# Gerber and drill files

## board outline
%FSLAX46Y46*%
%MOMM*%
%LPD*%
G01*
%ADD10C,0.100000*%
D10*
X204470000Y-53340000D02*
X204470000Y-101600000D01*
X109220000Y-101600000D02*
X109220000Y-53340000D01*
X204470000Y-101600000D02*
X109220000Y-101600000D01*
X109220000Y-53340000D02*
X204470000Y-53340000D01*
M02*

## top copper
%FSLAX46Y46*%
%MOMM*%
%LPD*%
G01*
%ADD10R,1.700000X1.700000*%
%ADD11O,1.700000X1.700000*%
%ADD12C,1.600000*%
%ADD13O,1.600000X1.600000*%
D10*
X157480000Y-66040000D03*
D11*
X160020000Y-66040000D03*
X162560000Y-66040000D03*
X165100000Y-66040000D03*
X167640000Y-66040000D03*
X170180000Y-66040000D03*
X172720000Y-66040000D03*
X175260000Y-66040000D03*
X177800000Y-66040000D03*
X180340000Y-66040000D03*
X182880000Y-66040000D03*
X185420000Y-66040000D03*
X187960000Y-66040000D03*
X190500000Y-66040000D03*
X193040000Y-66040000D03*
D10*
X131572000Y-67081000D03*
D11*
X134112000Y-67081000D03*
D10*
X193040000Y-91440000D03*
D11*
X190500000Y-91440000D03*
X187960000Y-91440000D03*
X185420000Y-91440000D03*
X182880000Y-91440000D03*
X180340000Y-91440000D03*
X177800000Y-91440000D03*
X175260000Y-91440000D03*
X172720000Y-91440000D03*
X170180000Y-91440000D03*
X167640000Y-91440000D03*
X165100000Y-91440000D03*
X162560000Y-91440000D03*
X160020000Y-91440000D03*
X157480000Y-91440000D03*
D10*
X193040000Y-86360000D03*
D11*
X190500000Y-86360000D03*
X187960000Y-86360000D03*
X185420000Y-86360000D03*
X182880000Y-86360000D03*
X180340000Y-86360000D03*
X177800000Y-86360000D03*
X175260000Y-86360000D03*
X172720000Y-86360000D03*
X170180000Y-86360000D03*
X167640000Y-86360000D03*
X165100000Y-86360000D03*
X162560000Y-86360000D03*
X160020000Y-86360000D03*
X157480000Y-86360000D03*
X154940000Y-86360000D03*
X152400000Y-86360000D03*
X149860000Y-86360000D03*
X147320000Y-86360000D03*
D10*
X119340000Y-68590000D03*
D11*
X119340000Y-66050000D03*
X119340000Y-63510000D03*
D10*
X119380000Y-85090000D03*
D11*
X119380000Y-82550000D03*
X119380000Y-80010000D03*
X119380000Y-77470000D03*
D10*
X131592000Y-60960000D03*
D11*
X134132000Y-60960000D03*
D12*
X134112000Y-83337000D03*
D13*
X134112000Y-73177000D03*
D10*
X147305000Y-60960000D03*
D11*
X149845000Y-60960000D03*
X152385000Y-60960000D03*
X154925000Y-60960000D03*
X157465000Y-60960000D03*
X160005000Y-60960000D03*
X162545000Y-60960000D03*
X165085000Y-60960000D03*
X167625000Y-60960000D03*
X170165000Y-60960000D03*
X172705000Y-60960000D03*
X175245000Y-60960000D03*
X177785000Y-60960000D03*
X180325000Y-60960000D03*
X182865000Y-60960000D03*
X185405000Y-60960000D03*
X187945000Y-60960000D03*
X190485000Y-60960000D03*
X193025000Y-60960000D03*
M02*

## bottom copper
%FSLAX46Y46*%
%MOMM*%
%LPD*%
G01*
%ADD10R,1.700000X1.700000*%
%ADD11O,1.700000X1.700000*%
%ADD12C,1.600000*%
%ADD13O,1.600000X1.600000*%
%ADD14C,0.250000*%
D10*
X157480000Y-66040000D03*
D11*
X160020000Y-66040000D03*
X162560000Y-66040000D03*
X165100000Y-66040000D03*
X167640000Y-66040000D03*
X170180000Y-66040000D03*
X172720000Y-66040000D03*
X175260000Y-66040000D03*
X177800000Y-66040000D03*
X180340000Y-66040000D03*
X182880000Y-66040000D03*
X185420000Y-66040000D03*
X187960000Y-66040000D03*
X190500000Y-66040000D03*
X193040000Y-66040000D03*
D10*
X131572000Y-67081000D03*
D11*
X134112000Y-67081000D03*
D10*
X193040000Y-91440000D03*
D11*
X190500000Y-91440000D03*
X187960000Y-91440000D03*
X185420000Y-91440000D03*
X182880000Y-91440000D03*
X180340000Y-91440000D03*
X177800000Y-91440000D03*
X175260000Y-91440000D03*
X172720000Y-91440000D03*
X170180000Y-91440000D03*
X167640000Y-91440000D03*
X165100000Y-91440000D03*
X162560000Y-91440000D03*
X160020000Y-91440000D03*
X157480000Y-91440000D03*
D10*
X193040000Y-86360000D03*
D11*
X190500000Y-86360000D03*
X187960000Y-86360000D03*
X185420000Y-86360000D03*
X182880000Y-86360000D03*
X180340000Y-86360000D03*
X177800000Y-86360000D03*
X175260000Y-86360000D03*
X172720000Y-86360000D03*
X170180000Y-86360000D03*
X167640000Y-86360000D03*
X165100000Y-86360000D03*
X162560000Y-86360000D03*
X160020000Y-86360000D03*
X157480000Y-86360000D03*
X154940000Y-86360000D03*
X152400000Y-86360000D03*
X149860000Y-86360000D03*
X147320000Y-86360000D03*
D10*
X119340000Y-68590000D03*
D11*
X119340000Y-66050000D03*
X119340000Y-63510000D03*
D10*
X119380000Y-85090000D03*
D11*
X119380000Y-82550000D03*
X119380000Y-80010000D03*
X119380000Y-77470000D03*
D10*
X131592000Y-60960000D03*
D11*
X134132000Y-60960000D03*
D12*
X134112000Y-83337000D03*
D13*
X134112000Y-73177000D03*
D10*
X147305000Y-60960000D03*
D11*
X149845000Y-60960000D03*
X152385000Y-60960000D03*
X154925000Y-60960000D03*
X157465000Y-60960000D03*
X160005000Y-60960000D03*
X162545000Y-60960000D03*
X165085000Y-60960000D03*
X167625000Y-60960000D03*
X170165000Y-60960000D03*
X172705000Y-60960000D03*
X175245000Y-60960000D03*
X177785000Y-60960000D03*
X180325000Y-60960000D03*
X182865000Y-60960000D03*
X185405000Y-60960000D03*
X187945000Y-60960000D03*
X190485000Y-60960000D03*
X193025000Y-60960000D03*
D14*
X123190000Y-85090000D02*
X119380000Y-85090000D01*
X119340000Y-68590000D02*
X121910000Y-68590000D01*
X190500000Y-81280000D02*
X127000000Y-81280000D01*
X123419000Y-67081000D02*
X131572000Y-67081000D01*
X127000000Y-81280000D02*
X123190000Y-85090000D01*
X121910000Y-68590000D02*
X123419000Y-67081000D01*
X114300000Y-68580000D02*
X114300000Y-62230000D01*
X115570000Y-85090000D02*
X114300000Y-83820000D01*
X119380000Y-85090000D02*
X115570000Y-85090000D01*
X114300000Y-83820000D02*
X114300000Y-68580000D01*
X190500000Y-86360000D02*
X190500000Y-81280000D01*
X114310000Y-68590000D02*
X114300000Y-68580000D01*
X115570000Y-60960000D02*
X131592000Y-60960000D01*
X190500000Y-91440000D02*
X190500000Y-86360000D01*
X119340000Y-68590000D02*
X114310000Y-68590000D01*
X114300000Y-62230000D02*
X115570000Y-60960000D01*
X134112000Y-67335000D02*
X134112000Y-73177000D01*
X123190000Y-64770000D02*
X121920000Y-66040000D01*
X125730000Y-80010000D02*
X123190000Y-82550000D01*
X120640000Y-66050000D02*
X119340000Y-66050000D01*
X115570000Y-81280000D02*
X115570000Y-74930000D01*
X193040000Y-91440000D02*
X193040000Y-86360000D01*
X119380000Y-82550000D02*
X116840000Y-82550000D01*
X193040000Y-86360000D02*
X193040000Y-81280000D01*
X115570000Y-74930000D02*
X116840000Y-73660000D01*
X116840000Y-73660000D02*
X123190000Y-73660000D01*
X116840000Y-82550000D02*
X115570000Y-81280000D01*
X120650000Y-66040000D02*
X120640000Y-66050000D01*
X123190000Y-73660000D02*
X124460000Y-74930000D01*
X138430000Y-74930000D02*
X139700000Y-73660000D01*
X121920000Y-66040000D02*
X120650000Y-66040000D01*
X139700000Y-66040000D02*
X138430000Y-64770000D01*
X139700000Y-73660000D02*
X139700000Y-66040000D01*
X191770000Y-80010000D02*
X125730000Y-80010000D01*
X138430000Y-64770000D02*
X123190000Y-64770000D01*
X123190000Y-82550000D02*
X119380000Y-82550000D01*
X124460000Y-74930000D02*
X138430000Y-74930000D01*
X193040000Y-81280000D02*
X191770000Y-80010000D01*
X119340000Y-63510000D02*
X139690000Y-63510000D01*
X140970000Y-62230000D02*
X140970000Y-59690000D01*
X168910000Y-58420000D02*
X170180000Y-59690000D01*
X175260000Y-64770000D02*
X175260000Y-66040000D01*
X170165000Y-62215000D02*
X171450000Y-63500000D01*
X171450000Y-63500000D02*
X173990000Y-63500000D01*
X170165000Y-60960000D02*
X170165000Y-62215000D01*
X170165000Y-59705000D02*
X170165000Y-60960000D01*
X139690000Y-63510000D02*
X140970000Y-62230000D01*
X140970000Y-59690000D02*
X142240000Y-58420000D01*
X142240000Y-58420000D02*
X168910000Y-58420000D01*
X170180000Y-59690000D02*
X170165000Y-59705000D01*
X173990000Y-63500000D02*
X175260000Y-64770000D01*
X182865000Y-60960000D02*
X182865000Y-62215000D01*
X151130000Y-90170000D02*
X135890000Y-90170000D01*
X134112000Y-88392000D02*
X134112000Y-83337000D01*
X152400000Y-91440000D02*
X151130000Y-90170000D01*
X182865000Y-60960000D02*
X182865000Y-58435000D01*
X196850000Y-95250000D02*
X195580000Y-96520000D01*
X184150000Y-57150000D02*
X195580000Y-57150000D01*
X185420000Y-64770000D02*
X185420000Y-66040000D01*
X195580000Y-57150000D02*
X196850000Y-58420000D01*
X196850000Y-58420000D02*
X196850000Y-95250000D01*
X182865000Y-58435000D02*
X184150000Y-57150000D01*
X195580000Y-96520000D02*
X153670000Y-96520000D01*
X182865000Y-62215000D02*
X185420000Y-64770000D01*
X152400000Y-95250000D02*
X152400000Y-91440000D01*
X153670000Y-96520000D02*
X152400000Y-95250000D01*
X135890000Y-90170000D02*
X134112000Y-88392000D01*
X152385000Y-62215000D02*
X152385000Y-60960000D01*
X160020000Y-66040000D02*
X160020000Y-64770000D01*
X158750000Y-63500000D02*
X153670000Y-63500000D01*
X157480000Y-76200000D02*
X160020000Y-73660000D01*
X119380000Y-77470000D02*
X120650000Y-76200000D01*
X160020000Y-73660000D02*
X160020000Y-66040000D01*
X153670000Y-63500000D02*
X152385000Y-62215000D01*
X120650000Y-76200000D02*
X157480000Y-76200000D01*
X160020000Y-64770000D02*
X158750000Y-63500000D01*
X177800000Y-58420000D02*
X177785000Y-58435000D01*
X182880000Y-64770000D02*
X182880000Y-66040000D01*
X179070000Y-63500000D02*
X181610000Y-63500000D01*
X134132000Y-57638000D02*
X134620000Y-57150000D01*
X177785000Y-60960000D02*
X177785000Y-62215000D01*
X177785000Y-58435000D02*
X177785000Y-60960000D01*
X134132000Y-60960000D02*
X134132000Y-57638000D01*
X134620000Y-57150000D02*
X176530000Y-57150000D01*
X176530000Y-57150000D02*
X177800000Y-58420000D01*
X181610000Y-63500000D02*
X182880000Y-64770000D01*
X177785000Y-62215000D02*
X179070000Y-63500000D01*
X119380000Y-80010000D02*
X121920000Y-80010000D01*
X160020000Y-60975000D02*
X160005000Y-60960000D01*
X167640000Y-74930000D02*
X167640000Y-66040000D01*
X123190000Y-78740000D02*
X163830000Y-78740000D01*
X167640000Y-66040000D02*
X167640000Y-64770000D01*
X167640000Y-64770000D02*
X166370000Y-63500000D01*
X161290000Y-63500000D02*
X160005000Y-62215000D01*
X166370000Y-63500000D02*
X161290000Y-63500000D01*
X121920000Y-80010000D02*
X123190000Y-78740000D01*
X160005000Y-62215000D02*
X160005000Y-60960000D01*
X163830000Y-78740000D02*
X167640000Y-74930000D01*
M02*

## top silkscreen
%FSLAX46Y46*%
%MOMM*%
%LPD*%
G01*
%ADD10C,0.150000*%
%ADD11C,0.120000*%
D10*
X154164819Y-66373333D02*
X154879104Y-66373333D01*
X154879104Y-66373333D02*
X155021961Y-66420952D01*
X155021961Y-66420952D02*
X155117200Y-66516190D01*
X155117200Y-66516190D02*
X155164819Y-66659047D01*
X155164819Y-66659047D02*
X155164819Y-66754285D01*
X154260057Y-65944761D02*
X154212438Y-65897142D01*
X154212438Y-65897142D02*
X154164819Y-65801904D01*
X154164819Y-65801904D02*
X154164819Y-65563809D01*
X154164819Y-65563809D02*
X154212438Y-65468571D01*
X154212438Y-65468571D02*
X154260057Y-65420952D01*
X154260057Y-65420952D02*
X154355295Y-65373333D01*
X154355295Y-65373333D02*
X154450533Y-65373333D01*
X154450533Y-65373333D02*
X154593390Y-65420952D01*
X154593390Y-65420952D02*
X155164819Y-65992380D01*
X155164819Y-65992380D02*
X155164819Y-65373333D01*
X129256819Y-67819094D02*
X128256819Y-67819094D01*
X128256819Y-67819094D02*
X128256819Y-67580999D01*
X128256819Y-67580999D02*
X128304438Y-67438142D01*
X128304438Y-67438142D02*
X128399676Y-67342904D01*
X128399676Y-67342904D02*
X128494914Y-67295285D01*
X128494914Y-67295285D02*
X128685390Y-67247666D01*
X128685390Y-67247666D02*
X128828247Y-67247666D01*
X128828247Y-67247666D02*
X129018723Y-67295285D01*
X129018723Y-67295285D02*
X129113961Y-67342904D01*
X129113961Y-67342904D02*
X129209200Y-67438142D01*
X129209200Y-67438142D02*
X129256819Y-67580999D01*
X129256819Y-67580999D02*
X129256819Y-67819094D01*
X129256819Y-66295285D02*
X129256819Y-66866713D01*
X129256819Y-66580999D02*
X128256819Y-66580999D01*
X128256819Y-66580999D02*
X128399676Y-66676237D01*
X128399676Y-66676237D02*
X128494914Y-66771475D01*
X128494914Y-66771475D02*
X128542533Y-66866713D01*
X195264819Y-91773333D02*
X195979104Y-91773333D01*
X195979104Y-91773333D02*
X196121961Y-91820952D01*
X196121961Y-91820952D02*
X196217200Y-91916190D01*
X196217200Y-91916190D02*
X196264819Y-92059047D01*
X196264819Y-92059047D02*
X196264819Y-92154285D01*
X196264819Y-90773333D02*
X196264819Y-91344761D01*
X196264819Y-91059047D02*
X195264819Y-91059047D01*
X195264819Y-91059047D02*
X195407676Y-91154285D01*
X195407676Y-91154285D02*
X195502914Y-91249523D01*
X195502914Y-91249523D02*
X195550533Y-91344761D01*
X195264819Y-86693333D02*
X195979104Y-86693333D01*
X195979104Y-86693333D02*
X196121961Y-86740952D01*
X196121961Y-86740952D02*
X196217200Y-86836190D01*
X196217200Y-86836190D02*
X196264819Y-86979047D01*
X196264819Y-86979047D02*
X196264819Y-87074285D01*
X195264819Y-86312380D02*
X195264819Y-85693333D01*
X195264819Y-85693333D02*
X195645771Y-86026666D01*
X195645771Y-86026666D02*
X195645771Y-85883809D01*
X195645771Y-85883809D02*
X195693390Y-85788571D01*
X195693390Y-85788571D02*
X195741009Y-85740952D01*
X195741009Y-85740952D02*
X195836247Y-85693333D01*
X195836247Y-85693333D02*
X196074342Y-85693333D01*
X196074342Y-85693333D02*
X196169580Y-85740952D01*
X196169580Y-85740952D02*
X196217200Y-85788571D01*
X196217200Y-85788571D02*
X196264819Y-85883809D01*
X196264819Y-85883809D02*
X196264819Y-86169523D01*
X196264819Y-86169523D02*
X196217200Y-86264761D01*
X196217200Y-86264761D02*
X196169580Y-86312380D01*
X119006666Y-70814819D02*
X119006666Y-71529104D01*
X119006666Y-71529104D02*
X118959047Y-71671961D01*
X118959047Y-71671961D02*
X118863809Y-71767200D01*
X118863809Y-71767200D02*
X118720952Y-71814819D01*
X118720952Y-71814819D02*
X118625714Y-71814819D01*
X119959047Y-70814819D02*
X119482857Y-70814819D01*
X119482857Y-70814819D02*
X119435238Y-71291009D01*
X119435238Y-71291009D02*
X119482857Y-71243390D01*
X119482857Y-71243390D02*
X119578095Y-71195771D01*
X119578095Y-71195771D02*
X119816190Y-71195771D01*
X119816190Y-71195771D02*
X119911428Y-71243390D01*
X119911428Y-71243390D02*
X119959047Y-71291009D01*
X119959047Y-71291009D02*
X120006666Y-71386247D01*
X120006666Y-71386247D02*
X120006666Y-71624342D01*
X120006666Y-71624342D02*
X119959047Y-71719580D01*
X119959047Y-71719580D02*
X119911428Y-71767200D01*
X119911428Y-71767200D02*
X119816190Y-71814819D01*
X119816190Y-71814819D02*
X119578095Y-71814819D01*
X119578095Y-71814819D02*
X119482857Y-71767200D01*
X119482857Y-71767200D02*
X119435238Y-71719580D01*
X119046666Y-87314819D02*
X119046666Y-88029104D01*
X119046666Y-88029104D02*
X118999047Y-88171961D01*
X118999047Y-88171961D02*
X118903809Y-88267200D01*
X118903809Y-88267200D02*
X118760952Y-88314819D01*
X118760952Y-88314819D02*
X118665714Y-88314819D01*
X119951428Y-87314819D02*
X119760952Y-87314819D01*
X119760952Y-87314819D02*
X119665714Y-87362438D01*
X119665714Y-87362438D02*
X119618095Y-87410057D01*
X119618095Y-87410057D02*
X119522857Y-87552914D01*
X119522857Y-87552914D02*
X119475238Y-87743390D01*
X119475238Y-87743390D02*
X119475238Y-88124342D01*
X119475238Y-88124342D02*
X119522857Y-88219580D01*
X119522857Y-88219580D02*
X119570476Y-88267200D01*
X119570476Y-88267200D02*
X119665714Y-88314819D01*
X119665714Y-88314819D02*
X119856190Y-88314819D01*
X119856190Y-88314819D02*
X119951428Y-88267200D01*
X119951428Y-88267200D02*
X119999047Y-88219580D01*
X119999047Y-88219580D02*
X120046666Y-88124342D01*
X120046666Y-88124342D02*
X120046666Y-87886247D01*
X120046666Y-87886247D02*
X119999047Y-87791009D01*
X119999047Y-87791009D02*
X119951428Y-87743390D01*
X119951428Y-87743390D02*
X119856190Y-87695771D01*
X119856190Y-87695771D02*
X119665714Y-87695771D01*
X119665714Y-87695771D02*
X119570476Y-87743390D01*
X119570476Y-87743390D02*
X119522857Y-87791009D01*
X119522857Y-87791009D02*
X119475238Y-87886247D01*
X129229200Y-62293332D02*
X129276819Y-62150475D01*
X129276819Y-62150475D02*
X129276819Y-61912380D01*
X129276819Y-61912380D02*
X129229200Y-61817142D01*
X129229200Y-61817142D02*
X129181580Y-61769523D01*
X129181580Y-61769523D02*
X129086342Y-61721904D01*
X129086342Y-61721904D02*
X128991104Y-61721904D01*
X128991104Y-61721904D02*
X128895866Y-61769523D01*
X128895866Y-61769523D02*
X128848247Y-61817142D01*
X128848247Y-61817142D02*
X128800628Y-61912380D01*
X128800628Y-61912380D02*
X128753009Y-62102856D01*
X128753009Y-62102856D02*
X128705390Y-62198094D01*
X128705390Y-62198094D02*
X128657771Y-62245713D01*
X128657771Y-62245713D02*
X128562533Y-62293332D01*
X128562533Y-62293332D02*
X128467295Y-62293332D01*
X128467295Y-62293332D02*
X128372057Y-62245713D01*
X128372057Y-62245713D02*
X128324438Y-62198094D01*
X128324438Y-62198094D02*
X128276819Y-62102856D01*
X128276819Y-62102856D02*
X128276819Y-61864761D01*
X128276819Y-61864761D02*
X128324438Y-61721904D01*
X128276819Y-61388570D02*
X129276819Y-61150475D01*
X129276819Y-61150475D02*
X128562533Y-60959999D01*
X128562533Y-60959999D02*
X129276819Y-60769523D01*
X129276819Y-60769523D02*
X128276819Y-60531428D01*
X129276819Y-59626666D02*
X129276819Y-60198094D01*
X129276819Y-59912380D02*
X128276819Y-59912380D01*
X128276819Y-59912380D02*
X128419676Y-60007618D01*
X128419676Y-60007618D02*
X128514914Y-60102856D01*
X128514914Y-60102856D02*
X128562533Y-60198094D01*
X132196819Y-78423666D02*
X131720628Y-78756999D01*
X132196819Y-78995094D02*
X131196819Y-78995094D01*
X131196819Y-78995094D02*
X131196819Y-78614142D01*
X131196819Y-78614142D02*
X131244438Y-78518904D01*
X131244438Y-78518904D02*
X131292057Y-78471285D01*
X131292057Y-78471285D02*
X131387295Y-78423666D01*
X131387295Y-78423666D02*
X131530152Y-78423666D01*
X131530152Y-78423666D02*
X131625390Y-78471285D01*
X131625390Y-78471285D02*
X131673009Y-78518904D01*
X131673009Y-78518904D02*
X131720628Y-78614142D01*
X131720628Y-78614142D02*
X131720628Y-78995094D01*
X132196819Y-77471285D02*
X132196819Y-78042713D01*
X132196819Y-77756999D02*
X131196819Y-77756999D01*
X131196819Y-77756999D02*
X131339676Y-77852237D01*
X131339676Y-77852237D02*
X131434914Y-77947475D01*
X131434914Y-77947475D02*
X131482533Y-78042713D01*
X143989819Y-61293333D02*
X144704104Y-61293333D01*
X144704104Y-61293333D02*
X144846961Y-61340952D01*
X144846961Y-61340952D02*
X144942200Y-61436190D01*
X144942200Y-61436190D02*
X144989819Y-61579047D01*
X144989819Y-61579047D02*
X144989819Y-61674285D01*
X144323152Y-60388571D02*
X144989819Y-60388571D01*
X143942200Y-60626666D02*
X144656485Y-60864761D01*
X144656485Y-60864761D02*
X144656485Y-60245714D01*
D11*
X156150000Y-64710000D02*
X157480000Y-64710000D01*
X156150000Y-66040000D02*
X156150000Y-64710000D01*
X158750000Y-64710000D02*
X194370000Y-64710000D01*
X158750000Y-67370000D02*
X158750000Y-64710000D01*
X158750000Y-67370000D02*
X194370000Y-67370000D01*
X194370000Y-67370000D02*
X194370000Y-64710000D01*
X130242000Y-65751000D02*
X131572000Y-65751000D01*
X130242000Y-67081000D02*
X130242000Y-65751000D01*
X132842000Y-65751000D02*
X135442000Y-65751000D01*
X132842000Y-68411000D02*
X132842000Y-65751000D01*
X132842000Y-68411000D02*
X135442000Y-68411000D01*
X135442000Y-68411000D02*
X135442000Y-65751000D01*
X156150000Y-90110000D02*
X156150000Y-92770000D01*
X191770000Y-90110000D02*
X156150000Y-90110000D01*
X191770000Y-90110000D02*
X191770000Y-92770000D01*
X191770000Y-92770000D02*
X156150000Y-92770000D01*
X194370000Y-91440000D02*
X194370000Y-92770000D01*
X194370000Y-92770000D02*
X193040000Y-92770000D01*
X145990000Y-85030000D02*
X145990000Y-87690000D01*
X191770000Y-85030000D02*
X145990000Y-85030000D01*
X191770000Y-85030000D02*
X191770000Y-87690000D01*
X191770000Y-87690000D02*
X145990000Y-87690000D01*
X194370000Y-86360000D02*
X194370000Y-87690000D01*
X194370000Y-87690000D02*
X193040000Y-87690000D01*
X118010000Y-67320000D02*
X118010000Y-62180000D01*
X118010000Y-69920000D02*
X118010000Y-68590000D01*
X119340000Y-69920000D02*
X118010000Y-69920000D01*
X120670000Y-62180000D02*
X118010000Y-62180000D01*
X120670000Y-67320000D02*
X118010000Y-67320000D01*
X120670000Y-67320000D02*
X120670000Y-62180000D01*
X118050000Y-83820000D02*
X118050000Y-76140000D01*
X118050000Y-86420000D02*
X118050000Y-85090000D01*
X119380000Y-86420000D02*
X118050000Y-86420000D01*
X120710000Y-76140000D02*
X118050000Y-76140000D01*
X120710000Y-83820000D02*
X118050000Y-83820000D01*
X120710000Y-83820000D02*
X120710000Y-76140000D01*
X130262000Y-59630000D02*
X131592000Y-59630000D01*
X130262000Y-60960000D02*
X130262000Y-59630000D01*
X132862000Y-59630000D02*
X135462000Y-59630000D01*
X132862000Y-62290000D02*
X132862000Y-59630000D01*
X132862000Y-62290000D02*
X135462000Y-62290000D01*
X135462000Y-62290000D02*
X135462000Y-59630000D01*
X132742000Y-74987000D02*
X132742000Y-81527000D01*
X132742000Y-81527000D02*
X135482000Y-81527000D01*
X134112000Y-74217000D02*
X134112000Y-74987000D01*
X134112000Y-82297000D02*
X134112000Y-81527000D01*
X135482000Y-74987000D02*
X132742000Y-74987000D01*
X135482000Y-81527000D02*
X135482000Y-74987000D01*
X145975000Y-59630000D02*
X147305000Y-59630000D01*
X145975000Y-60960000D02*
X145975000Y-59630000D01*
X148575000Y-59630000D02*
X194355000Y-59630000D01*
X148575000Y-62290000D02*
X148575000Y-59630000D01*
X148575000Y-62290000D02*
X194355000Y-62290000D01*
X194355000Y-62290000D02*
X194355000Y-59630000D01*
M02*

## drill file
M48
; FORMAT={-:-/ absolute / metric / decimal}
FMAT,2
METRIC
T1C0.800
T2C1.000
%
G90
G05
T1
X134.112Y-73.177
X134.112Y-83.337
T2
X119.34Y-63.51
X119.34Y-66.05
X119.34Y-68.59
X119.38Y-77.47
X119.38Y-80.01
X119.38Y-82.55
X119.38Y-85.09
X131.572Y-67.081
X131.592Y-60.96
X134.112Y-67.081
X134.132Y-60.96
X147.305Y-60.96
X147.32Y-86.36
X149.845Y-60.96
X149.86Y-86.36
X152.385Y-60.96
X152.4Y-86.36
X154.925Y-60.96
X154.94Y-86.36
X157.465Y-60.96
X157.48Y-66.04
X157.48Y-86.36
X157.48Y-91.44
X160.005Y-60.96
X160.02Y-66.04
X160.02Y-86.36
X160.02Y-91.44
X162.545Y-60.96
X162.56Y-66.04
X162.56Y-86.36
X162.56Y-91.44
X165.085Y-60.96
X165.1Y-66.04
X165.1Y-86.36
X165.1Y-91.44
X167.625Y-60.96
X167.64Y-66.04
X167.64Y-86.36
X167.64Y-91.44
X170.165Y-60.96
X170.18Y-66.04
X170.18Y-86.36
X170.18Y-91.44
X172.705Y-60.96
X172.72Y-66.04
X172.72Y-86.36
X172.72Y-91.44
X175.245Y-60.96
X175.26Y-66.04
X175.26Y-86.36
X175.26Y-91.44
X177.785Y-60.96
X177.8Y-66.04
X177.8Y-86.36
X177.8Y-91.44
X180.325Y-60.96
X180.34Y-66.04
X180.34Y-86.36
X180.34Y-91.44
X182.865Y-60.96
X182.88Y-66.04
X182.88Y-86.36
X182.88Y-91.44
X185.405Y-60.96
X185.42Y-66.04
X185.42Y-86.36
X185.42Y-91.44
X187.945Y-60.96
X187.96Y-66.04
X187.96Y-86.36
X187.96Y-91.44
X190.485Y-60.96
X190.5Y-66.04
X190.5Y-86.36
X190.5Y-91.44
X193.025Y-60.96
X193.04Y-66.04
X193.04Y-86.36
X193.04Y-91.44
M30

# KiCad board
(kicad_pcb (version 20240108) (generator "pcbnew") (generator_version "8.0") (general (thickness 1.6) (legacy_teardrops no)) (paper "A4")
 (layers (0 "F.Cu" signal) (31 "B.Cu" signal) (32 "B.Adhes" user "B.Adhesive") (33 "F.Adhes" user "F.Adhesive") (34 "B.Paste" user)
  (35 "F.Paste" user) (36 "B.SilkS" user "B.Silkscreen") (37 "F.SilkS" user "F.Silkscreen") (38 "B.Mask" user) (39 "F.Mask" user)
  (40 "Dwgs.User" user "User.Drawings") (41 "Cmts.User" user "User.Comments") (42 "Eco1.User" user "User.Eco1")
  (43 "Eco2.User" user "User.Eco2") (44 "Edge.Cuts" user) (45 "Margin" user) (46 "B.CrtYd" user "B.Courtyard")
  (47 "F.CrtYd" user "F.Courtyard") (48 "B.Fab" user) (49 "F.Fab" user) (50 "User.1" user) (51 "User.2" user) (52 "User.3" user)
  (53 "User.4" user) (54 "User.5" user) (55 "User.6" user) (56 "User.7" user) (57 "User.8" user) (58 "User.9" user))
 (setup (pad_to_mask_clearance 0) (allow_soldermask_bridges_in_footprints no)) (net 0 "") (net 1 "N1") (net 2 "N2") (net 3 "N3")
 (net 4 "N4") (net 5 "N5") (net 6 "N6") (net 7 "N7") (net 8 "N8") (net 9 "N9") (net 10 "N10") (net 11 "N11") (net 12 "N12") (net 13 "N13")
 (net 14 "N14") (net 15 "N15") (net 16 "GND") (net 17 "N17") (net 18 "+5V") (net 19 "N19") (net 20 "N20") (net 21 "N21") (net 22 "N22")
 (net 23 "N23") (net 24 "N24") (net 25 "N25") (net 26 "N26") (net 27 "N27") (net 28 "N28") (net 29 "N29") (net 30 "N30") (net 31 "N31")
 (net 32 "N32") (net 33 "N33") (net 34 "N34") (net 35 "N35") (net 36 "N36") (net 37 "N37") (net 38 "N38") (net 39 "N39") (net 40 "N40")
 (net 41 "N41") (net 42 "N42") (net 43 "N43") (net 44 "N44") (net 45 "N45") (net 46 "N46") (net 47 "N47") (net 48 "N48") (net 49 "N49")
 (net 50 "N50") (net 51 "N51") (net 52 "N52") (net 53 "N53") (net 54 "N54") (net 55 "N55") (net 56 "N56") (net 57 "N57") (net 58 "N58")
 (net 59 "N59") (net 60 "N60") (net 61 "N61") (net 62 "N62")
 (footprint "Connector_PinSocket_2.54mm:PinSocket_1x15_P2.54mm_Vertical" (layer "F.Cu") (at 157.48 66.04 90)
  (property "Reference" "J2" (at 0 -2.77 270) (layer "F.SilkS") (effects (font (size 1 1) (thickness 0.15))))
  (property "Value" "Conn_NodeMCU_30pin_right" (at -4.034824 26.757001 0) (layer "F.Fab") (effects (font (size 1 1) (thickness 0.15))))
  (fp_line (start 1.33 -1.33) (end 1.33 0) (stroke (width 0.12) (type solid)) (layer "F.SilkS"))
  (fp_line (start 0 -1.33) (end 1.33 -1.33) (stroke (width 0.12) (type solid)) (layer "F.SilkS"))
  (fp_line (start 1.33 1.27) (end 1.33 36.89) (stroke (width 0.12) (type solid)) (layer "F.SilkS"))
  (fp_line (start -1.33 1.27) (end 1.33 1.27) (stroke (width 0.12) (type solid)) (layer "F.SilkS"))
  (fp_line (start -1.33 1.27) (end -1.33 36.89) (stroke (width 0.12) (type solid)) (layer "F.SilkS"))
  (fp_line (start -1.33 36.89) (end 1.33 36.89) (stroke (width 0.12) (type solid)) (layer "F.SilkS"))
  (pad "1" thru_hole rect (at 0 0 90) (size 1.7 1.7) (drill 1) (layers "*.Cu" "*.Mask") (remove_unused_layers no) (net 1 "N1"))
  (pad "2" thru_hole oval (at 0 2.54 90) (size 1.7 1.7) (drill 1) (layers "*.Cu" "*.Mask") (remove_unused_layers no) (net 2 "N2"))
  (pad "3" thru_hole oval (at 0 5.08 90) (size 1.7 1.7) (drill 1) (layers "*.Cu" "*.Mask") (remove_unused_layers no) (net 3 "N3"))
  (pad "4" thru_hole oval (at 0 7.62 90) (size 1.7 1.7) (drill 1) (layers "*.Cu" "*.Mask") (remove_unused_layers no) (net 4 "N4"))
  (pad "5" thru_hole oval (at 0 10.16 90) (size 1.7 1.7) (drill 1) (layers "*.Cu" "*.Mask") (remove_unused_layers no) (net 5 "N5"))
  (pad "6" thru_hole oval (at 0 12.7 90) (size 1.7 1.7) (drill 1) (layers "*.Cu" "*.Mask") (remove_unused_layers no) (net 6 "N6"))
  (pad "7" thru_hole oval (at 0 15.24 90) (size 1.7 1.7) (drill 1) (layers "*.Cu" "*.Mask") (remove_unused_layers no) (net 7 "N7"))
  (pad "8" thru_hole oval (at 0 17.78 90) (size 1.7 1.7) (drill 1) (layers "*.Cu" "*.Mask") (remove_unused_layers no) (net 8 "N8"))
  (pad "9" thru_hole oval (at 0 20.32 90) (size 1.7 1.7) (drill 1) (layers "*.Cu" "*.Mask") (remove_unused_layers no) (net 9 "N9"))
  (pad "10" thru_hole oval (at 0 22.86 90) (size 1.7 1.7) (drill 1) (layers "*.Cu" "*.Mask") (remove_unused_layers no) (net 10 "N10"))
  (pad "11" thru_hole oval (at 0 25.4 90) (size 1.7 1.7) (drill 1) (layers "*.Cu" "*.Mask") (remove_unused_layers no) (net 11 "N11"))
  (pad "12" thru_hole oval (at 0 27.94 90) (size 1.7 1.7) (drill 1) (layers "*.Cu" "*.Mask") (remove_unused_layers no) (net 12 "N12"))
  (pad "13" thru_hole oval (at 0 30.48 90) (size 1.7 1.7) (drill 1) (layers "*.Cu" "*.Mask") (remove_unused_layers no) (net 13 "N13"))
  (pad "14" thru_hole oval (at 0 33.02 90) (size 1.7 1.7) (drill 1) (layers "*.Cu" "*.Mask") (remove_unused_layers no) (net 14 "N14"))
  (pad "15" thru_hole oval (at 0 35.56 90) (size 1.7 1.7) (drill 1) (layers "*.Cu" "*.Mask") (remove_unused_layers no) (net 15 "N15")))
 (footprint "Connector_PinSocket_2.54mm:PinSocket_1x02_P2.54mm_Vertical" (layer "F.Cu") (at 131.572 67.081 90)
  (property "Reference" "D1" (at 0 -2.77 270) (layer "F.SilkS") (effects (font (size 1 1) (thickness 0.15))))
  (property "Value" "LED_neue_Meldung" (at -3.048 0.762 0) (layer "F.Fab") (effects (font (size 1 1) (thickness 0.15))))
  (fp_line (start 1.33 -1.33) (end 1.33 0) (stroke (width 0.12) (type solid)) (layer "F.SilkS"))
  (fp_line (start 0 -1.33) (end 1.33 -1.33) (stroke (width 0.12) (type solid)) (layer "F.SilkS"))
  (fp_line (start 1.33 1.27) (end 1.33 3.87) (stroke (width 0.12) (type solid)) (layer "F.SilkS"))
  (fp_line (start -1.33 1.27) (end 1.33 1.27) (stroke (width 0.12) (type solid)) (layer "F.SilkS"))
  (fp_line (start -1.33 1.27) (end -1.33 3.87) (stroke (width 0.12) (type solid)) (layer "F.SilkS"))
  (fp_line (start -1.33 3.87) (end 1.33 3.87) (stroke (width 0.12) (type solid)) (layer "F.SilkS"))
  (pad "1" thru_hole rect (at 0 0 90) (size 1.7 1.7) (drill 1) (layers "*.Cu" "*.Mask") (remove_unused_layers no) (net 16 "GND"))
  (pad "2" thru_hole oval (at 0 2.54 90) (size 1.7 1.7) (drill 1) (layers "*.Cu" "*.Mask") (remove_unused_layers no) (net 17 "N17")))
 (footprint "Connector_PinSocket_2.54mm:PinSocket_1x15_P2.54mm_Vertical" (layer "F.Cu") (at 193.04 91.44 -90)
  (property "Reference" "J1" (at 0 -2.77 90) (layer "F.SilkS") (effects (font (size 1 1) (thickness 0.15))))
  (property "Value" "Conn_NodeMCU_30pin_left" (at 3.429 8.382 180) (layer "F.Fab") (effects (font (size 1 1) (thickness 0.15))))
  (fp_line (start -1.33 36.89) (end 1.33 36.89) (stroke (width 0.12) (type solid)) (layer "F.SilkS"))
  (fp_line (start -1.33 1.27) (end -1.33 36.89) (stroke (width 0.12) (type solid)) (layer "F.SilkS"))
  (fp_line (start -1.33 1.27) (end 1.33 1.27) (stroke (width 0.12) (type solid)) (layer "F.SilkS"))
  (fp_line (start 1.33 1.27) (end 1.33 36.89) (stroke (width 0.12) (type solid)) (layer "F.SilkS"))
  (fp_line (start 0 -1.33) (end 1.33 -1.33) (stroke (width 0.12) (type solid)) (layer "F.SilkS"))
  (fp_line (start 1.33 -1.33) (end 1.33 0) (stroke (width 0.12) (type solid)) (layer "F.SilkS"))
  (pad "1" thru_hole rect (at 0 0 270) (size 1.7 1.7) (drill 1) (layers "*.Cu" "*.Mask") (remove_unused_layers no) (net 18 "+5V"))
  (pad "2" thru_hole oval (at 0 2.54 270) (size 1.7 1.7) (drill 1) (layers "*.Cu" "*.Mask") (remove_unused_layers no) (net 16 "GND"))
  (pad "3" thru_hole oval (at 0 5.08 270) (size 1.7 1.7) (drill 1) (layers "*.Cu" "*.Mask") (remove_unused_layers no) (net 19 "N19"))
  (pad "4" thru_hole oval (at 0 7.62 270) (size 1.7 1.7) (drill 1) (layers "*.Cu" "*.Mask") (remove_unused_layers no) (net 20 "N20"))
  (pad "5" thru_hole oval (at 0 10.16 270) (size 1.7 1.7) (drill 1) (layers "*.Cu" "*.Mask") (remove_unused_layers no) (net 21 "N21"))
  (pad "6" thru_hole oval (at 0 12.7 270) (size 1.7 1.7) (drill 1) (layers "*.Cu" "*.Mask") (remove_unused_layers no) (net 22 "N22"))
  (pad "7" thru_hole oval (at 0 15.24 270) (size 1.7 1.7) (drill 1) (layers "*.Cu" "*.Mask") (remove_unused_layers no) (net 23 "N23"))
  (pad "8" thru_hole oval (at 0 17.78 270) (size 1.7 1.7) (drill 1) (layers "*.Cu" "*.Mask") (remove_unused_layers no) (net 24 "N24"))
  (pad "9" thru_hole oval (at 0 20.32 270) (size 1.7 1.7) (drill 1) (layers "*.Cu" "*.Mask") (remove_unused_layers no) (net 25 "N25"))
  (pad "10" thru_hole oval (at 0 22.86 270) (size 1.7 1.7) (drill 1) (layers "*.Cu" "*.Mask") (remove_unused_layers no) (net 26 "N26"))
  (pad "11" thru_hole oval (at 0 25.4 270) (size 1.7 1.7) (drill 1) (layers "*.Cu" "*.Mask") (remove_unused_layers no) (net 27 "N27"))
  (pad "12" thru_hole oval (at 0 27.94 270) (size 1.7 1.7) (drill 1) (layers "*.Cu" "*.Mask") (remove_unused_layers no) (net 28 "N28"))
  (pad "13" thru_hole oval (at 0 30.48 270) (size 1.7 1.7) (drill 1) (layers "*.Cu" "*.Mask") (remove_unused_layers no) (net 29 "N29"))
  (pad "14" thru_hole oval (at 0 33.02 270) (size 1.7 1.7) (drill 1) (layers "*.Cu" "*.Mask") (remove_unused_layers no) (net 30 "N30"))
  (pad "15" thru_hole oval (at 0 35.56 270) (size 1.7 1.7) (drill 1) (layers "*.Cu" "*.Mask") (remove_unused_layers no) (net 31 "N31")))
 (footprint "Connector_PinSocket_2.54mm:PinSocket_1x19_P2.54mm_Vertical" (layer "F.Cu") (at 193.04 86.36 -90)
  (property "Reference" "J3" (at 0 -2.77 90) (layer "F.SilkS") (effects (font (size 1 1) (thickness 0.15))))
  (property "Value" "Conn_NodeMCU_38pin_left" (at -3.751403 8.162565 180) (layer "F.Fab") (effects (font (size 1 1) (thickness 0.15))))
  (fp_line (start -1.33 47.05) (end 1.33 47.05) (stroke (width 0.12) (type solid)) (layer "F.SilkS"))
  (fp_line (start -1.33 1.27) (end -1.33 47.05) (stroke (width 0.12) (type solid)) (layer "F.SilkS"))
  (fp_line (start -1.33 1.27) (end 1.33 1.27) (stroke (width 0.12) (type solid)) (layer "F.SilkS"))
  (fp_line (start 1.33 1.27) (end 1.33 47.05) (stroke (width 0.12) (type solid)) (layer "F.SilkS"))
  (fp_line (start 0 -1.33) (end 1.33 -1.33) (stroke (width 0.12) (type solid)) (layer "F.SilkS"))
  (fp_line (start 1.33 -1.33) (end 1.33 0) (stroke (width 0.12) (type solid)) (layer "F.SilkS"))
  (pad "1" thru_hole rect (at 0 0 270) (size 1.7 1.7) (drill 1) (layers "*.Cu" "*.Mask") (remove_unused_layers no) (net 18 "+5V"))
  (pad "2" thru_hole oval (at 0 2.54 270) (size 1.7 1.7) (drill 1) (layers "*.Cu" "*.Mask") (remove_unused_layers no) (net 16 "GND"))
  (pad "3" thru_hole oval (at 0 5.08 270) (size 1.7 1.7) (drill 1) (layers "*.Cu" "*.Mask") (remove_unused_layers no) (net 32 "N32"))
  (pad "4" thru_hole oval (at 0 7.62 270) (size 1.7 1.7) (drill 1) (layers "*.Cu" "*.Mask") (remove_unused_layers no) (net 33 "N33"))
  (pad "5" thru_hole oval (at 0 10.16 270) (size 1.7 1.7) (drill 1) (layers "*.Cu" "*.Mask") (remove_unused_layers no) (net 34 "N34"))
  (pad "6" thru_hole oval (at 0 12.7 270) (size 1.7 1.7) (drill 1) (layers "*.Cu" "*.Mask") (remove_unused_layers no) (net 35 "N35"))
  (pad "7" thru_hole oval (at 0 15.24 270) (size 1.7 1.7) (drill 1) (layers "*.Cu" "*.Mask") (remove_unused_layers no) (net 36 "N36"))
  (pad "8" thru_hole oval (at 0 17.78 270) (size 1.7 1.7) (drill 1) (layers "*.Cu" "*.Mask") (remove_unused_layers no) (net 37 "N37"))
  (pad "9" thru_hole oval (at 0 20.32 270) (size 1.7 1.7) (drill 1) (layers "*.Cu" "*.Mask") (remove_unused_layers no) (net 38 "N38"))
  (pad "10" thru_hole oval (at 0 22.86 270) (size 1.7 1.7) (drill 1) (layers "*.Cu" "*.Mask") (remove_unused_layers no) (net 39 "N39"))
  (pad "11" thru_hole oval (at 0 25.4 270) (size 1.7 1.7) (drill 1) (layers "*.Cu" "*.Mask") (remove_unused_layers no) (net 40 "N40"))
  (pad "12" thru_hole oval (at 0 27.94 270) (size 1.7 1.7) (drill 1) (layers "*.Cu" "*.Mask") (remove_unused_layers no) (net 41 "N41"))
  (pad "13" thru_hole oval (at 0 30.48 270) (size 1.7 1.7) (drill 1) (layers "*.Cu" "*.Mask") (remove_unused_layers no) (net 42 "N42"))
  (pad "14" thru_hole oval (at 0 33.02 270) (size 1.7 1.7) (drill 1) (layers "*.Cu" "*.Mask") (remove_unused_layers no) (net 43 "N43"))
  (pad "15" thru_hole oval (at 0 35.56 270) (size 1.7 1.7) (drill 1) (layers "*.Cu" "*.Mask") (remove_unused_layers no) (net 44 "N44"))
  (pad "16" thru_hole oval (at 0 38.1 270) (size 1.7 1.7) (drill 1) (layers "*.Cu" "*.Mask") (remove_unused_layers no) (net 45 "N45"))
  (pad "17" thru_hole oval (at 0 40.64 270) (size 1.7 1.7) (drill 1) (layers "*.Cu" "*.Mask") (remove_unused_layers no) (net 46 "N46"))
  (pad "18" thru_hole oval (at 0 43.18 270) (size 1.7 1.7) (drill 1) (layers "*.Cu" "*.Mask") (remove_unused_layers no) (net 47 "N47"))
  (pad "19" thru_hole oval (at 0 45.72 270) (size 1.7 1.7) (drill 1) (layers "*.Cu" "*.Mask") (remove_unused_layers no) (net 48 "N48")))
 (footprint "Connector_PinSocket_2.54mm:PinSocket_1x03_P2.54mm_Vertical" (layer "F.Cu") (at 119.34 68.59 180)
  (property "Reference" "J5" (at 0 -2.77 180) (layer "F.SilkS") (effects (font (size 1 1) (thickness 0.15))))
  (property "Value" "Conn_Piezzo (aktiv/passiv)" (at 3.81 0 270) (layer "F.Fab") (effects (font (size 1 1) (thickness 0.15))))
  (fp_line (start 1.33 1.27) (end 1.33 6.41) (stroke (width 0.12) (type solid)) (layer "F.SilkS"))
  (fp_line (start 1.33 -1.33) (end 1.33 0) (stroke (width 0.12) (type solid)) (layer "F.SilkS"))
  (fp_line (start 0 -1.33) (end 1.33 -1.33) (stroke (width 0.12) (type solid)) (layer "F.SilkS"))
  (fp_line (start -1.33 6.41) (end 1.33 6.41) (stroke (width 0.12) (type solid)) (layer "F.SilkS"))
  (fp_line (start -1.33 1.27) (end 1.33 1.27) (stroke (width 0.12) (type solid)) (layer "F.SilkS"))
  (fp_line (start -1.33 1.27) (end -1.33 6.41) (stroke (width 0.12) (type solid)) (layer "F.SilkS"))
  (pad "1" thru_hole rect (at 0 0 180) (size 1.7 1.7) (drill 1) (layers "*.Cu" "*.Mask") (remove_unused_layers no) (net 16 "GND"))
  (pad "2" thru_hole oval (at 0 2.54 180) (size 1.7 1.7) (drill 1) (layers "*.Cu" "*.Mask") (remove_unused_layers no) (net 18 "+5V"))
  (pad "3" thru_hole oval (at 0 5.08 180) (size 1.7 1.7) (drill 1) (layers "*.Cu" "*.Mask") (remove_unused_layers no) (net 8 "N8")))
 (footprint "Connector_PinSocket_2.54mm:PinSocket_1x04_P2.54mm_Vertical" (layer "F.Cu") (at 119.38 85.09 180)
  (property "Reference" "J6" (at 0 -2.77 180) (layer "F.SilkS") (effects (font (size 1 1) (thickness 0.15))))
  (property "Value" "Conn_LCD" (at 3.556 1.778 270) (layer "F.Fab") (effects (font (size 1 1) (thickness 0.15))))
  (fp_line (start 1.33 1.27) (end 1.33 8.95) (stroke (width 0.12) (type solid)) (layer "F.SilkS"))
  (fp_line (start 1.33 -1.33) (end 1.33 0) (stroke (width 0.12) (type solid)) (layer "F.SilkS"))
  (fp_line (start 0 -1.33) (end 1.33 -1.33) (stroke (width 0.12) (type solid)) (layer "F.SilkS"))
  (fp_line (start -1.33 8.95) (end 1.33 8.95) (stroke (width 0.12) (type solid)) (layer "F.SilkS"))
  (fp_line (start -1.33 1.27) (end 1.33 1.27) (stroke (width 0.12) (type solid)) (layer "F.SilkS"))
  (fp_line (start -1.33 1.27) (end -1.33 8.95) (stroke (width 0.12) (type solid)) (layer "F.SilkS"))
  (pad "1" thru_hole rect (at 0 0 180) (size 1.7 1.7) (drill 1) (layers "*.Cu" "*.Mask") (remove_unused_layers no) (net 16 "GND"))
  (pad "2" thru_hole oval (at 0 2.54 180) (size 1.7 1.7) (drill 1) (layers "*.Cu" "*.Mask") (remove_unused_layers no) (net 18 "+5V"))
  (pad "3" thru_hole oval (at 0 5.08 180) (size 1.7 1.7) (drill 1) (layers "*.Cu" "*.Mask") (remove_unused_layers no) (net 5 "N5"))
  (pad "4" thru_hole oval (at 0 7.62 180) (size 1.7 1.7) (drill 1) (layers "*.Cu" "*.Mask") (remove_unused_layers no) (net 2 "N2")))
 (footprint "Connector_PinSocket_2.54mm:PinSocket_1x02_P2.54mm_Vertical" (layer "F.Cu") (at 131.592 60.96 90)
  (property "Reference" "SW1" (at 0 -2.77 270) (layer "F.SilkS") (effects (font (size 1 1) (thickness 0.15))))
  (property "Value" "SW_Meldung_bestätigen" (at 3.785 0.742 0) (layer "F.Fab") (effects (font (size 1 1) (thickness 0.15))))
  (fp_line (start 1.33 -1.33) (end 1.33 0) (stroke (width 0.12) (type solid)) (layer "F.SilkS"))
  (fp_line (start 0 -1.33) (end 1.33 -1.33) (stroke (width 0.12) (type solid)) (layer "F.SilkS"))
  (fp_line (start 1.33 1.27) (end 1.33 3.87) (stroke (width 0.12) (type solid)) (layer "F.SilkS"))
  (fp_line (start -1.33 1.27) (end 1.33 1.27) (stroke (width 0.12) (type solid)) (layer "F.SilkS"))
  (fp_line (start -1.33 1.27) (end -1.33 3.87) (stroke (width 0.12) (type solid)) (layer "F.SilkS"))
  (fp_line (start -1.33 3.87) (end 1.33 3.87) (stroke (width 0.12) (type solid)) (layer "F.SilkS"))
  (pad "1" thru_hole rect (at 0 0 90) (size 1.7 1.7) (drill 1) (layers "*.Cu" "*.Mask") (remove_unused_layers no) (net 16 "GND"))
  (pad "2" thru_hole oval (at 0 2.54 90) (size 1.7 1.7) (drill 1) (layers "*.Cu" "*.Mask") (remove_unused_layers no) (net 11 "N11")))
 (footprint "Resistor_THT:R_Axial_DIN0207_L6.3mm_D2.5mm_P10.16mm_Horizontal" (layer "F.Cu") (at 134.112 83.337 90)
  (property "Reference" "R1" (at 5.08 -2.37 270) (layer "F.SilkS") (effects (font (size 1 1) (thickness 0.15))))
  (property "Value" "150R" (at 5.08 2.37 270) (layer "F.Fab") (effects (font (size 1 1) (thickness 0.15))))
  (fp_line (start 8.35 -1.37) (end 1.81 -1.37) (stroke (width 0.12) (type solid)) (layer "F.SilkS"))
  (fp_line (start 1.81 -1.37) (end 1.81 1.37) (stroke (width 0.12) (type solid)) (layer "F.SilkS"))
  (fp_line (start 9.12 0) (end 8.35 0) (stroke (width 0.12) (type solid)) (layer "F.SilkS"))
  (fp_line (start 1.04 0) (end 1.81 0) (stroke (width 0.12) (type solid)) (layer "F.SilkS"))
  (fp_line (start 8.35 1.37) (end 8.35 -1.37) (stroke (width 0.12) (type solid)) (layer "F.SilkS"))
  (fp_line (start 1.81 1.37) (end 8.35 1.37) (stroke (width 0.12) (type solid)) (layer "F.SilkS"))
  (pad "1" thru_hole circle (at 0 0 90) (size 1.6 1.6) (drill 0.8) (layers "*.Cu" "*.Mask") (remove_unused_layers no) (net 12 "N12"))
  (pad "2" thru_hole oval (at 10.16 0 90) (size 1.6 1.6) (drill 0.8) (layers "*.Cu" "*.Mask") (remove_unused_layers no) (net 17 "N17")))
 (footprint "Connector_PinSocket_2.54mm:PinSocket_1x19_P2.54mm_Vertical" (layer "F.Cu") (at 147.305 60.96 90)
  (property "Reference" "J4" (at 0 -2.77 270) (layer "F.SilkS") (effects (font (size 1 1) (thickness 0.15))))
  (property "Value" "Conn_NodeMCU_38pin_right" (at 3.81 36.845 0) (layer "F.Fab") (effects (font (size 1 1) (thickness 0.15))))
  (fp_line (start 1.33 -1.33) (end 1.33 0) (stroke (width 0.12) (type solid)) (layer "F.SilkS"))
  (fp_line (start 0 -1.33) (end 1.33 -1.33) (stroke (width 0.12) (type solid)) (layer "F.SilkS"))
  (fp_line (start 1.33 1.27) (end 1.33 47.05) (stroke (width 0.12) (type solid)) (layer "F.SilkS"))
  (fp_line (start -1.33 1.27) (end 1.33 1.27) (stroke (width 0.12) (type solid)) (layer "F.SilkS"))
  (fp_line (start -1.33 1.27) (end -1.33 47.05) (stroke (width 0.12) (type solid)) (layer "F.SilkS"))
  (fp_line (start -1.33 47.05) (end 1.33 47.05) (stroke (width 0.12) (type solid)) (layer "F.SilkS"))
  (pad "1" thru_hole rect (at 0 0 90) (size 1.7 1.7) (drill 1) (layers "*.Cu" "*.Mask") (remove_unused_layers no) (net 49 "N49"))
  (pad "2" thru_hole oval (at 0 2.54 90) (size 1.7 1.7) (drill 1) (layers "*.Cu" "*.Mask") (remove_unused_layers no) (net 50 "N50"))
  (pad "3" thru_hole oval (at 0 5.08 90) (size 1.7 1.7) (drill 1) (layers "*.Cu" "*.Mask") (remove_unused_layers no) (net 2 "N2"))
  (pad "4" thru_hole oval (at 0 7.62 90) (size 1.7 1.7) (drill 1) (layers "*.Cu" "*.Mask") (remove_unused_layers no) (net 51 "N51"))
  (pad "5" thru_hole oval (at 0 10.16 90) (size 1.7 1.7) (drill 1) (layers "*.Cu" "*.Mask") (remove_unused_layers no) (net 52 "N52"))
  (pad "6" thru_hole oval (at 0 12.7 90) (size 1.7 1.7) (drill 1) (layers "*.Cu" "*.Mask") (remove_unused_layers no) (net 5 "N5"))
  (pad "7" thru_hole oval (at 0 15.24 90) (size 1.7 1.7) (drill 1) (layers "*.Cu" "*.Mask") (remove_unused_layers no) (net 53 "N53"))
  (pad "8" thru_hole oval (at 0 17.78 90) (size 1.7 1.7) (drill 1) (layers "*.Cu" "*.Mask") (remove_unused_layers no) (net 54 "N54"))
  (pad "9" thru_hole oval (at 0 20.32 90) (size 1.7 1.7) (drill 1) (layers "*.Cu" "*.Mask") (remove_unused_layers no) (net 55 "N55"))
  (pad "10" thru_hole oval (at 0 22.86 90) (size 1.7 1.7) (drill 1) (layers "*.Cu" "*.Mask") (remove_unused_layers no) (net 8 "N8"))
  (pad "11" thru_hole oval (at 0 25.4 90) (size 1.7 1.7) (drill 1) (layers "*.Cu" "*.Mask") (remove_unused_layers no) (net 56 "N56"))
  (pad "12" thru_hole oval (at 0 27.94 90) (size 1.7 1.7) (drill 1) (layers "*.Cu" "*.Mask") (remove_unused_layers no) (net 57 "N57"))
  (pad "13" thru_hole oval (at 0 30.48 90) (size 1.7 1.7) (drill 1) (layers "*.Cu" "*.Mask") (remove_unused_layers no) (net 11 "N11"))
  (pad "14" thru_hole oval (at 0 33.02 90) (size 1.7 1.7) (drill 1) (layers "*.Cu" "*.Mask") (remove_unused_layers no) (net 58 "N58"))
  (pad "15" thru_hole oval (at 0 35.56 90) (size 1.7 1.7) (drill 1) (layers "*.Cu" "*.Mask") (remove_unused_layers no) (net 12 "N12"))
  (pad "16" thru_hole oval (at 0 38.1 90) (size 1.7 1.7) (drill 1) (layers "*.Cu" "*.Mask") (remove_unused_layers no) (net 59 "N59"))
  (pad "17" thru_hole oval (at 0 40.64 90) (size 1.7 1.7) (drill 1) (layers "*.Cu" "*.Mask") (remove_unused_layers no) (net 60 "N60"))
  (pad "18" thru_hole oval (at 0 43.18 90) (size 1.7 1.7) (drill 1) (layers "*.Cu" "*.Mask") (remove_unused_layers no) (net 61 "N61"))
  (pad "19" thru_hole oval (at 0 45.72 90) (size 1.7 1.7) (drill 1) (layers "*.Cu" "*.Mask") (remove_unused_layers no) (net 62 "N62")))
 (gr_line (start 204.47 53.34) (end 204.47 101.6) (stroke (width 0.1) (type default)) (layer "Edge.Cuts"))
 (gr_line (start 109.22 101.6) (end 109.22 53.34) (stroke (width 0.1) (type default)) (layer "Edge.Cuts"))
 (gr_line (start 204.47 101.6) (end 109.22 101.6) (stroke (width 0.1) (type default)) (layer "Edge.Cuts"))
 (gr_line (start 109.22 53.34) (end 204.47 53.34) (stroke (width 0.1) (type default)) (layer "Edge.Cuts"))
 (segment (start 123.19 85.09) (end 119.38 85.09) (width 0.25) (layer "B.Cu") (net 16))
 (segment (start 119.34 68.59) (end 121.91 68.59) (width 0.25) (layer "B.Cu") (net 16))
 (segment (start 190.5 81.28) (end 127 81.28) (width 0.25) (layer "B.Cu") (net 16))
 (segment (start 123.419 67.081) (end 131.572 67.081) (width 0.25) (layer "B.Cu") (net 16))
 (segment (start 127 81.28) (end 123.19 85.09) (width 0.25) (layer "B.Cu") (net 16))
 (segment (start 121.91 68.59) (end 123.419 67.081) (width 0.25) (layer "B.Cu") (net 16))
 (segment (start 114.3 68.58) (end 114.3 62.23) (width 0.25) (layer "B.Cu") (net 16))
 (segment (start 115.57 85.09) (end 114.3 83.82) (width 0.25) (layer "B.Cu") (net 16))
 (segment (start 119.38 85.09) (end 115.57 85.09) (width 0.25) (layer "B.Cu") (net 16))
 (segment (start 114.3 83.82) (end 114.3 68.58) (width 0.25) (layer "B.Cu") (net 16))
 (segment (start 190.5 86.36) (end 190.5 81.28) (width 0.25) (layer "B.Cu") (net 16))
 (segment (start 114.31 68.59) (end 114.3 68.58) (width 0.25) (layer "B.Cu") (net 16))
 (segment (start 115.57 60.96) (end 131.592 60.96) (width 0.25) (layer "B.Cu") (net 16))
 (segment (start 190.5 91.44) (end 190.5 86.36) (width 0.25) (layer "B.Cu") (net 16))
 (segment (start 119.34 68.59) (end 114.31 68.59) (width 0.25) (layer "B.Cu") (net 16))
 (segment (start 114.3 62.23) (end 115.57 60.96) (width 0.25) (layer "B.Cu") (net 16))
 (segment (start 134.112 67.335) (end 134.112 73.177) (width 0.25) (layer "B.Cu") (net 17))
 (segment (start 123.19 64.77) (end 121.92 66.04) (width 0.25) (layer "B.Cu") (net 18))
 (segment (start 125.73 80.01) (end 123.19 82.55) (width 0.25) (layer "B.Cu") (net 18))
 (segment (start 120.64 66.05) (end 119.34 66.05) (width 0.25) (layer "B.Cu") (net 18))
 (segment (start 115.57 81.28) (end 115.57 74.93) (width 0.25) (layer "B.Cu") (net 18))
 (segment (start 193.04 91.44) (end 193.04 86.36) (width 0.25) (layer "B.Cu") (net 18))
 (segment (start 119.38 82.55) (end 116.84 82.55) (width 0.25) (layer "B.Cu") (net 18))
 (segment (start 193.04 86.36) (end 193.04 81.28) (width 0.25) (layer "B.Cu") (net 18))
 (segment (start 115.57 74.93) (end 116.84 73.66) (width 0.25) (layer "B.Cu") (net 18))
 (segment (start 116.84 73.66) (end 123.19 73.66) (width 0.25) (layer "B.Cu") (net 18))
 (segment (start 116.84 82.55) (end 115.57 81.28) (width 0.25) (layer "B.Cu") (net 18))
 (segment (start 120.65 66.04) (end 120.64 66.05) (width 0.25) (layer "B.Cu") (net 18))
 (segment (start 123.19 73.66) (end 124.46 74.93) (width 0.25) (layer "B.Cu") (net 18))
 (segment (start 138.43 74.93) (end 139.7 73.66) (width 0.25) (layer "B.Cu") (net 18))
 (segment (start 121.92 66.04) (end 120.65 66.04) (width 0.25) (layer "B.Cu") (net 18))
 (segment (start 139.7 66.04) (end 138.43 64.77) (width 0.25) (layer "B.Cu") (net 18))
 (segment (start 139.7 73.66) (end 139.7 66.04) (width 0.25) (layer "B.Cu") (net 18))
 (segment (start 191.77 80.01) (end 125.73 80.01) (width 0.25) (layer "B.Cu") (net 18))
 (segment (start 138.43 64.77) (end 123.19 64.77) (width 0.25) (layer "B.Cu") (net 18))
 (segment (start 123.19 82.55) (end 119.38 82.55) (width 0.25) (layer "B.Cu") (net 18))
 (segment (start 124.46 74.93) (end 138.43 74.93) (width 0.25) (layer "B.Cu") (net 18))
 (segment (start 193.04 81.28) (end 191.77 80.01) (width 0.25) (layer "B.Cu") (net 18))
 (segment (start 119.34 63.51) (end 139.69 63.51) (width 0.25) (layer "B.Cu") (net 8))
 (segment (start 140.97 62.23) (end 140.97 59.69) (width 0.25) (layer "B.Cu") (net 8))
 (segment (start 168.91 58.42) (end 170.18 59.69) (width 0.25) (layer "B.Cu") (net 8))
 (segment (start 175.26 64.77) (end 175.26 66.04) (width 0.25) (layer "B.Cu") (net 8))
 (segment (start 170.165 62.215) (end 171.45 63.5) (width 0.25) (layer "B.Cu") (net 8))
 (segment (start 171.45 63.5) (end 173.99 63.5) (width 0.25) (layer "B.Cu") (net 8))
 (segment (start 170.165 60.96) (end 170.165 62.215) (width 0.25) (layer "B.Cu") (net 8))
 (segment (start 170.165 59.705) (end 170.165 60.96) (width 0.25) (layer "B.Cu") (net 8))
 (segment (start 139.69 63.51) (end 140.97 62.23) (width 0.25) (layer "B.Cu") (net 8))
 (segment (start 140.97 59.69) (end 142.24 58.42) (width 0.25) (layer "B.Cu") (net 8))
 (segment (start 142.24 58.42) (end 168.91 58.42) (width 0.25) (layer "B.Cu") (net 8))
 (segment (start 170.18 59.69) (end 170.165 59.705) (width 0.25) (layer "B.Cu") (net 8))
 (segment (start 173.99 63.5) (end 175.26 64.77) (width 0.25) (layer "B.Cu") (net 8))
 (segment (start 182.865 60.96) (end 182.865 62.215) (width 0.25) (layer "B.Cu") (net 12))
 (segment (start 151.13 90.17) (end 135.89 90.17) (width 0.25) (layer "B.Cu") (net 12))
 (segment (start 134.112 88.392) (end 134.112 83.337) (width 0.25) (layer "B.Cu") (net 12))
 (segment (start 152.4 91.44) (end 151.13 90.17) (width 0.25) (layer "B.Cu") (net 12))
 (segment (start 182.865 60.96) (end 182.865 58.435) (width 0.25) (layer "B.Cu") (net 12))
 (segment (start 196.85 95.25) (end 195.58 96.52) (width 0.25) (layer "B.Cu") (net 12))
 (segment (start 184.15 57.15) (end 195.58 57.15) (width 0.25) (layer "B.Cu") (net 12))
 (segment (start 185.42 64.77) (end 185.42 66.04) (width 0.25) (layer "B.Cu") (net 12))
 (segment (start 195.58 57.15) (end 196.85 58.42) (width 0.25) (layer "B.Cu") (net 12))
 (segment (start 196.85 58.42) (end 196.85 95.25) (width 0.25) (layer "B.Cu") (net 12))
 (segment (start 182.865 58.435) (end 184.15 57.15) (width 0.25) (layer "B.Cu") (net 12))
 (segment (start 195.58 96.52) (end 153.67 96.52) (width 0.25) (layer "B.Cu") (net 12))
 (segment (start 182.865 62.215) (end 185.42 64.77) (width 0.25) (layer "B.Cu") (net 12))
 (segment (start 152.4 95.25) (end 152.4 91.44) (width 0.25) (layer "B.Cu") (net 12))
 (segment (start 153.67 96.52) (end 152.4 95.25) (width 0.25) (layer "B.Cu") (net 12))
 (segment (start 135.89 90.17) (end 134.112 88.392) (width 0.25) (layer "B.Cu") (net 12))
 (segment (start 152.385 62.215) (end 152.385 60.96) (width 0.25) (layer "B.Cu") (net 2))
 (segment (start 160.02 66.04) (end 160.02 64.77) (width 0.25) (layer "B.Cu") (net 2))
 (segment (start 158.75 63.5) (end 153.67 63.5) (width 0.25) (layer "B.Cu") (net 2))
 (segment (start 157.48 76.2) (end 160.02 73.66) (width 0.25) (layer "B.Cu") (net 2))
 (segment (start 119.38 77.47) (end 120.65 76.2) (width 0.25) (layer "B.Cu") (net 2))
 (segment (start 160.02 73.66) (end 160.02 66.04) (width 0.25) (layer "B.Cu") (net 2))
 (segment (start 153.67 63.5) (end 152.385 62.215) (width 0.25) (layer "B.Cu") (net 2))
 (segment (start 120.65 76.2) (end 157.48 76.2) (width 0.25) (layer "B.Cu") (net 2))
 (segment (start 160.02 64.77) (end 158.75 63.5) (width 0.25) (layer "B.Cu") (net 2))
 (segment (start 177.8 58.42) (end 177.785 58.435) (width 0.25) (layer "B.Cu") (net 11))
 (segment (start 182.88 64.77) (end 182.88 66.04) (width 0.25) (layer "B.Cu") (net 11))
 (segment (start 179.07 63.5) (end 181.61 63.5) (width 0.25) (layer "B.Cu") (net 11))
 (segment (start 134.132 57.638) (end 134.62 57.15) (width 0.25) (layer "B.Cu") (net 11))
 (segment (start 177.785 60.96) (end 177.785 62.215) (width 0.25) (layer "B.Cu") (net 11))
 (segment (start 177.785 58.435) (end 177.785 60.96) (width 0.25) (layer "B.Cu") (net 11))
 (segment (start 134.132 60.96) (end 134.132 57.638) (width 0.25) (layer "B.Cu") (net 11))
 (segment (start 134.62 57.15) (end 176.53 57.15) (width 0.25) (layer "B.Cu") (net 11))
 (segment (start 176.53 57.15) (end 177.8 58.42) (width 0.25) (layer "B.Cu") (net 11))
 (segment (start 181.61 63.5) (end 182.88 64.77) (width 0.25) (layer "B.Cu") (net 11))
 (segment (start 177.785 62.215) (end 179.07 63.5) (width 0.25) (layer "B.Cu") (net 11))
 (segment (start 119.38 80.01) (end 121.92 80.01) (width 0.25) (layer "B.Cu") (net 5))
 (segment (start 160.02 60.975) (end 160.005 60.96) (width 0.25) (layer "B.Cu") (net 5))
 (segment (start 167.64 74.93) (end 167.64 66.04) (width 0.25) (layer "B.Cu") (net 5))
 (segment (start 123.19 78.74) (end 163.83 78.74) (width 0.25) (layer "B.Cu") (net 5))
 (segment (start 167.64 66.04) (end 167.64 64.77) (width 0.25) (layer "B.Cu") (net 5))
 (segment (start 167.64 64.77) (end 166.37 63.5) (width 0.25) (layer "B.Cu") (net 5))
 (segment (start 161.29 63.5) (end 160.005 62.215) (width 0.25) (layer "B.Cu") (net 5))
 (segment (start 166.37 63.5) (end 161.29 63.5) (width 0.25) (layer "B.Cu") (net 5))
 (segment (start 121.92 80.01) (end 123.19 78.74) (width 0.25) (layer "B.Cu") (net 5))
 (segment (start 160.005 62.215) (end 160.005 60.96) (width 0.25) (layer "B.Cu") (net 5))
 (segment (start 163.83 78.74) (end 167.64 74.93) (width 0.25) (layer "B.Cu") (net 5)))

